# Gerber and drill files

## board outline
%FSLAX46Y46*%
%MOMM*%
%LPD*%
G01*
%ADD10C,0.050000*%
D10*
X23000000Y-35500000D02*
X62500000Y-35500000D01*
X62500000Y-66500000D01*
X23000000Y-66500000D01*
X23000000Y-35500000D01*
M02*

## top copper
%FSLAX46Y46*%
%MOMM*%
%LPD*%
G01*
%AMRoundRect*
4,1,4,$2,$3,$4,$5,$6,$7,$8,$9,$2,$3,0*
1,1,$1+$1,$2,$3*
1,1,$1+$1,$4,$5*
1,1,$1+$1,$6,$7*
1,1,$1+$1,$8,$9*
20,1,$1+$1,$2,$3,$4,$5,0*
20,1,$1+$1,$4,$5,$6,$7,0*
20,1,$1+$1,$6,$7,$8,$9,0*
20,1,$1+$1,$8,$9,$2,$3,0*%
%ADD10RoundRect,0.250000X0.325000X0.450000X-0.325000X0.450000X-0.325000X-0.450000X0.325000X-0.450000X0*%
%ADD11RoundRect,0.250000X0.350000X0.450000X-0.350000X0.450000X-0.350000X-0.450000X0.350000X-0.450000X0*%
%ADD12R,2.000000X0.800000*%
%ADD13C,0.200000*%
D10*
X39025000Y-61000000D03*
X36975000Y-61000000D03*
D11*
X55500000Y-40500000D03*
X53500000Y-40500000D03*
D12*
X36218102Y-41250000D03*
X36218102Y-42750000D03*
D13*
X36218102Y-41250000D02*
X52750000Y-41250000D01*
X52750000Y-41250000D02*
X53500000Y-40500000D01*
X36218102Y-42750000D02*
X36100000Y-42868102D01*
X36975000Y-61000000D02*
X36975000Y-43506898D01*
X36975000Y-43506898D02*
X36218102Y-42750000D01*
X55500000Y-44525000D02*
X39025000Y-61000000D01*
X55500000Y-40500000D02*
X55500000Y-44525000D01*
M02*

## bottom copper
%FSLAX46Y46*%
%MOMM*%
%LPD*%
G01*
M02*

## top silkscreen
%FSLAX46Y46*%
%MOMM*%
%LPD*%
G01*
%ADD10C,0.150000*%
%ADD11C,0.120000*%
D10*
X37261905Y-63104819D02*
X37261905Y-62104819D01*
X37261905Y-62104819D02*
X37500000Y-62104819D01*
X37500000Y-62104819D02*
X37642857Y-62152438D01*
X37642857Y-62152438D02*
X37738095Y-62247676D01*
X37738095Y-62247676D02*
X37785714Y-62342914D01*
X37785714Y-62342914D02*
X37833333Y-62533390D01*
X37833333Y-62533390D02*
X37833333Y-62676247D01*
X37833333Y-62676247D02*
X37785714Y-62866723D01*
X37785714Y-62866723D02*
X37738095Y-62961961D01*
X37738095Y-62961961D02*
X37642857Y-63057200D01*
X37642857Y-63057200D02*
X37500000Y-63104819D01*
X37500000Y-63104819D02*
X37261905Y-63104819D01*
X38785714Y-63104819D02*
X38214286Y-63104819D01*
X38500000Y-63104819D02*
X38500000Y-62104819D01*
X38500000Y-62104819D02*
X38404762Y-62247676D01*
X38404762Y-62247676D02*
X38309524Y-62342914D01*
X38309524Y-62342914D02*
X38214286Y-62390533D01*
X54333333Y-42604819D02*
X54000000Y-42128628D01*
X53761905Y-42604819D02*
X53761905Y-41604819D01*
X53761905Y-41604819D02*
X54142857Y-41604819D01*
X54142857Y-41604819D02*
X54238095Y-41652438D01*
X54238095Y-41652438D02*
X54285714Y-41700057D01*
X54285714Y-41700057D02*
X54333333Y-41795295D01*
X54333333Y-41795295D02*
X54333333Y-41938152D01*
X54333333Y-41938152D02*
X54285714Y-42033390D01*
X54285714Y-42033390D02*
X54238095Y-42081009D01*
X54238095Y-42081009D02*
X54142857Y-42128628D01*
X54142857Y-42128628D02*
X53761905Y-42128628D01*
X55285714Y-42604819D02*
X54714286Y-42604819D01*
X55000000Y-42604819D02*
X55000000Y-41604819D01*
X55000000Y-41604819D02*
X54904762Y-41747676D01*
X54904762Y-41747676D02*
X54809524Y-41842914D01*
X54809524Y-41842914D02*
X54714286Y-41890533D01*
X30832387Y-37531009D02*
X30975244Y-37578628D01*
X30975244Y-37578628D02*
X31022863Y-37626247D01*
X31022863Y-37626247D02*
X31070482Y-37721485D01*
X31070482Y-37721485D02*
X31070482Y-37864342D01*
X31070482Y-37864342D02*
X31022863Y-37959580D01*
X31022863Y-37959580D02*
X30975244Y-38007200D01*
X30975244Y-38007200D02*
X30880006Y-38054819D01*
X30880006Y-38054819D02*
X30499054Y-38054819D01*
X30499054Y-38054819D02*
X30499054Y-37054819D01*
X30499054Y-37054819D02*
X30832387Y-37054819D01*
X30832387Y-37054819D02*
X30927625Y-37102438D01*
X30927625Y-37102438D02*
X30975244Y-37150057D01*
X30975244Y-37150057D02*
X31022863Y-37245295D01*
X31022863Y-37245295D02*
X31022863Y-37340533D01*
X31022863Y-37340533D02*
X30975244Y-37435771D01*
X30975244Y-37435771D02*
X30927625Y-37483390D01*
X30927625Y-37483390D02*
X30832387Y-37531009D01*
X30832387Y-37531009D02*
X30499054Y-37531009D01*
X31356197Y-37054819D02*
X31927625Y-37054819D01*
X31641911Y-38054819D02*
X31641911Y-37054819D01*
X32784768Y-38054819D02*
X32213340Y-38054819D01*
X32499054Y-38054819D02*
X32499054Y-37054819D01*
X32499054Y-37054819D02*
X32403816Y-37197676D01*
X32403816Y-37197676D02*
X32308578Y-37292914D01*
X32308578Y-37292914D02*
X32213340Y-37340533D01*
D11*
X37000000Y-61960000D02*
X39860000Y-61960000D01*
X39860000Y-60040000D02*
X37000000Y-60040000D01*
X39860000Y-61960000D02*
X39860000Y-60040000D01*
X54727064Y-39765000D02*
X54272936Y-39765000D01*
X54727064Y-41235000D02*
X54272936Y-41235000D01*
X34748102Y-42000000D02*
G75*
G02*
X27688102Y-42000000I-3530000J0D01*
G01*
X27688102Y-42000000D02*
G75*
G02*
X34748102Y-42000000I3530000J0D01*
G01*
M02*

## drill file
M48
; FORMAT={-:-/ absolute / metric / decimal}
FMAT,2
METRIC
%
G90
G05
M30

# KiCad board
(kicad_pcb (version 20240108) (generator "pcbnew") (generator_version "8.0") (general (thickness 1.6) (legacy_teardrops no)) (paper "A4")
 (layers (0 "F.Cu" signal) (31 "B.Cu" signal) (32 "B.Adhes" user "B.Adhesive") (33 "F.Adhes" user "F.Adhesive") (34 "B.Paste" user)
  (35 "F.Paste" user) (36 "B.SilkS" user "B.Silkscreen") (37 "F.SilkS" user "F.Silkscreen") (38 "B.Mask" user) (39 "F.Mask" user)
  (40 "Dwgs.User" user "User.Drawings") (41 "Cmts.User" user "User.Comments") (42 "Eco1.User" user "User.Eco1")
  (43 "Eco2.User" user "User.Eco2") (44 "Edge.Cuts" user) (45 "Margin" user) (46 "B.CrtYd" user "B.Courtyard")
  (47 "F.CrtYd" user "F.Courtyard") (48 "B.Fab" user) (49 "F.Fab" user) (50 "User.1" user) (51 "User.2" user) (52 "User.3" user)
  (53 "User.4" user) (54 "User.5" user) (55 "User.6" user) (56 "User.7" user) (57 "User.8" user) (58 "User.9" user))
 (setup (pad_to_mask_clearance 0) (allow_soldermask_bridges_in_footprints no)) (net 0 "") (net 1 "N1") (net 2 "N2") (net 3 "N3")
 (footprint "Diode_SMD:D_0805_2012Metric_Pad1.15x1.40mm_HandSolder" (layer "F.Cu") (at 38 61 180)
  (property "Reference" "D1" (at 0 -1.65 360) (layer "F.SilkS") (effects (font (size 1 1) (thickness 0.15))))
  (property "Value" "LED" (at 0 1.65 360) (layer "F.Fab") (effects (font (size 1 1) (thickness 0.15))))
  (fp_line (start 1 -0.96) (end -1.86 -0.96) (stroke (width 0.12) (type solid)) (layer "F.SilkS"))
  (fp_line (start -1.86 0.96) (end 1 0.96) (stroke (width 0.12) (type solid)) (layer "F.SilkS"))
  (fp_line (start -1.86 -0.96) (end -1.86 0.96) (stroke (width 0.12) (type solid)) (layer "F.SilkS"))
  (pad "1" smd roundrect (at -1.025 0 180) (size 1.15 1.4) (layers "F.Cu" "F.Paste" "F.Mask") (roundrect_rratio 0.217391) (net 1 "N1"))
  (pad "2" smd roundrect (at 1.025 0 180) (size 1.15 1.4) (layers "F.Cu" "F.Paste" "F.Mask") (roundrect_rratio 0.217391) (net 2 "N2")))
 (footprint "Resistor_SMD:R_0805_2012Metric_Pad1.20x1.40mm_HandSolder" (layer "F.Cu") (at 54.5 40.5 180)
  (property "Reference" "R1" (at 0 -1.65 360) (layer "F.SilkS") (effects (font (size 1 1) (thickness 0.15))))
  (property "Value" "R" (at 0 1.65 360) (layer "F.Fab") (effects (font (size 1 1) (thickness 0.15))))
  (fp_line (start -0.227064 0.735) (end 0.227064 0.735) (stroke (width 0.12) (type solid)) (layer "F.SilkS"))
  (fp_line (start -0.227064 -0.735) (end 0.227064 -0.735) (stroke (width 0.12) (type solid)) (layer "F.SilkS"))
  (pad "1" smd roundrect (at -1 0 180) (size 1.2 1.4) (layers "F.Cu" "F.Paste" "F.Mask") (roundrect_rratio 0.208333) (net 1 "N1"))
  (pad "2" smd roundrect (at 1 0 180) (size 1.2 1.4) (layers "F.Cu" "F.Paste" "F.Mask") (roundrect_rratio 0.208333) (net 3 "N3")))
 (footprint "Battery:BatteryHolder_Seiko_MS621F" (layer "F.Cu") (at 36.218102 42)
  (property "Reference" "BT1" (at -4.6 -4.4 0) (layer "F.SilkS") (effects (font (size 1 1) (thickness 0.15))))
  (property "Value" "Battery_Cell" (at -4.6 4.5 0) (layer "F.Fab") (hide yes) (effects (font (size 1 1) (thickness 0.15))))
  (fp_circle (center -5 0) (end -1.47 0) (stroke (width 0.12) (type solid)) (fill none) (layer "F.SilkS"))
  (pad "1" smd rect (at 0 -0.75) (size 2 0.8) (layers "F.Cu" "F.Paste" "F.Mask") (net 3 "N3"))
  (pad "2" smd rect (at 0 0.75) (size 2 0.8) (layers "F.Cu" "F.Paste" "F.Mask") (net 2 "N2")))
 (gr_rect (start 23 35.5) (end 62.5 66.5) (stroke (width 0.05) (type default)) (fill none) (layer "Edge.Cuts"))
 (segment (start 36.218102 41.25) (end 52.75 41.25) (width 0.2) (layer "F.Cu") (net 3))
 (segment (start 52.75 41.25) (end 53.5 40.5) (width 0.2) (layer "F.Cu") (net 3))
 (segment (start 36.218102 42.75) (end 36.1 42.868102) (width 0.2) (layer "F.Cu") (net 2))
 (segment (start 36.975 61) (end 36.975 43.506898) (width 0.2) (layer "F.Cu") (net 2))
 (segment (start 36.975 43.506898) (end 36.218102 42.75) (width 0.2) (layer "F.Cu") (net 2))
 (segment (start 55.5 44.525) (end 39.025 61) (width 0.2) (layer "F.Cu") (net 1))
 (segment (start 55.5 40.5) (end 55.5 44.525) (width 0.2) (layer "F.Cu") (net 1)))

